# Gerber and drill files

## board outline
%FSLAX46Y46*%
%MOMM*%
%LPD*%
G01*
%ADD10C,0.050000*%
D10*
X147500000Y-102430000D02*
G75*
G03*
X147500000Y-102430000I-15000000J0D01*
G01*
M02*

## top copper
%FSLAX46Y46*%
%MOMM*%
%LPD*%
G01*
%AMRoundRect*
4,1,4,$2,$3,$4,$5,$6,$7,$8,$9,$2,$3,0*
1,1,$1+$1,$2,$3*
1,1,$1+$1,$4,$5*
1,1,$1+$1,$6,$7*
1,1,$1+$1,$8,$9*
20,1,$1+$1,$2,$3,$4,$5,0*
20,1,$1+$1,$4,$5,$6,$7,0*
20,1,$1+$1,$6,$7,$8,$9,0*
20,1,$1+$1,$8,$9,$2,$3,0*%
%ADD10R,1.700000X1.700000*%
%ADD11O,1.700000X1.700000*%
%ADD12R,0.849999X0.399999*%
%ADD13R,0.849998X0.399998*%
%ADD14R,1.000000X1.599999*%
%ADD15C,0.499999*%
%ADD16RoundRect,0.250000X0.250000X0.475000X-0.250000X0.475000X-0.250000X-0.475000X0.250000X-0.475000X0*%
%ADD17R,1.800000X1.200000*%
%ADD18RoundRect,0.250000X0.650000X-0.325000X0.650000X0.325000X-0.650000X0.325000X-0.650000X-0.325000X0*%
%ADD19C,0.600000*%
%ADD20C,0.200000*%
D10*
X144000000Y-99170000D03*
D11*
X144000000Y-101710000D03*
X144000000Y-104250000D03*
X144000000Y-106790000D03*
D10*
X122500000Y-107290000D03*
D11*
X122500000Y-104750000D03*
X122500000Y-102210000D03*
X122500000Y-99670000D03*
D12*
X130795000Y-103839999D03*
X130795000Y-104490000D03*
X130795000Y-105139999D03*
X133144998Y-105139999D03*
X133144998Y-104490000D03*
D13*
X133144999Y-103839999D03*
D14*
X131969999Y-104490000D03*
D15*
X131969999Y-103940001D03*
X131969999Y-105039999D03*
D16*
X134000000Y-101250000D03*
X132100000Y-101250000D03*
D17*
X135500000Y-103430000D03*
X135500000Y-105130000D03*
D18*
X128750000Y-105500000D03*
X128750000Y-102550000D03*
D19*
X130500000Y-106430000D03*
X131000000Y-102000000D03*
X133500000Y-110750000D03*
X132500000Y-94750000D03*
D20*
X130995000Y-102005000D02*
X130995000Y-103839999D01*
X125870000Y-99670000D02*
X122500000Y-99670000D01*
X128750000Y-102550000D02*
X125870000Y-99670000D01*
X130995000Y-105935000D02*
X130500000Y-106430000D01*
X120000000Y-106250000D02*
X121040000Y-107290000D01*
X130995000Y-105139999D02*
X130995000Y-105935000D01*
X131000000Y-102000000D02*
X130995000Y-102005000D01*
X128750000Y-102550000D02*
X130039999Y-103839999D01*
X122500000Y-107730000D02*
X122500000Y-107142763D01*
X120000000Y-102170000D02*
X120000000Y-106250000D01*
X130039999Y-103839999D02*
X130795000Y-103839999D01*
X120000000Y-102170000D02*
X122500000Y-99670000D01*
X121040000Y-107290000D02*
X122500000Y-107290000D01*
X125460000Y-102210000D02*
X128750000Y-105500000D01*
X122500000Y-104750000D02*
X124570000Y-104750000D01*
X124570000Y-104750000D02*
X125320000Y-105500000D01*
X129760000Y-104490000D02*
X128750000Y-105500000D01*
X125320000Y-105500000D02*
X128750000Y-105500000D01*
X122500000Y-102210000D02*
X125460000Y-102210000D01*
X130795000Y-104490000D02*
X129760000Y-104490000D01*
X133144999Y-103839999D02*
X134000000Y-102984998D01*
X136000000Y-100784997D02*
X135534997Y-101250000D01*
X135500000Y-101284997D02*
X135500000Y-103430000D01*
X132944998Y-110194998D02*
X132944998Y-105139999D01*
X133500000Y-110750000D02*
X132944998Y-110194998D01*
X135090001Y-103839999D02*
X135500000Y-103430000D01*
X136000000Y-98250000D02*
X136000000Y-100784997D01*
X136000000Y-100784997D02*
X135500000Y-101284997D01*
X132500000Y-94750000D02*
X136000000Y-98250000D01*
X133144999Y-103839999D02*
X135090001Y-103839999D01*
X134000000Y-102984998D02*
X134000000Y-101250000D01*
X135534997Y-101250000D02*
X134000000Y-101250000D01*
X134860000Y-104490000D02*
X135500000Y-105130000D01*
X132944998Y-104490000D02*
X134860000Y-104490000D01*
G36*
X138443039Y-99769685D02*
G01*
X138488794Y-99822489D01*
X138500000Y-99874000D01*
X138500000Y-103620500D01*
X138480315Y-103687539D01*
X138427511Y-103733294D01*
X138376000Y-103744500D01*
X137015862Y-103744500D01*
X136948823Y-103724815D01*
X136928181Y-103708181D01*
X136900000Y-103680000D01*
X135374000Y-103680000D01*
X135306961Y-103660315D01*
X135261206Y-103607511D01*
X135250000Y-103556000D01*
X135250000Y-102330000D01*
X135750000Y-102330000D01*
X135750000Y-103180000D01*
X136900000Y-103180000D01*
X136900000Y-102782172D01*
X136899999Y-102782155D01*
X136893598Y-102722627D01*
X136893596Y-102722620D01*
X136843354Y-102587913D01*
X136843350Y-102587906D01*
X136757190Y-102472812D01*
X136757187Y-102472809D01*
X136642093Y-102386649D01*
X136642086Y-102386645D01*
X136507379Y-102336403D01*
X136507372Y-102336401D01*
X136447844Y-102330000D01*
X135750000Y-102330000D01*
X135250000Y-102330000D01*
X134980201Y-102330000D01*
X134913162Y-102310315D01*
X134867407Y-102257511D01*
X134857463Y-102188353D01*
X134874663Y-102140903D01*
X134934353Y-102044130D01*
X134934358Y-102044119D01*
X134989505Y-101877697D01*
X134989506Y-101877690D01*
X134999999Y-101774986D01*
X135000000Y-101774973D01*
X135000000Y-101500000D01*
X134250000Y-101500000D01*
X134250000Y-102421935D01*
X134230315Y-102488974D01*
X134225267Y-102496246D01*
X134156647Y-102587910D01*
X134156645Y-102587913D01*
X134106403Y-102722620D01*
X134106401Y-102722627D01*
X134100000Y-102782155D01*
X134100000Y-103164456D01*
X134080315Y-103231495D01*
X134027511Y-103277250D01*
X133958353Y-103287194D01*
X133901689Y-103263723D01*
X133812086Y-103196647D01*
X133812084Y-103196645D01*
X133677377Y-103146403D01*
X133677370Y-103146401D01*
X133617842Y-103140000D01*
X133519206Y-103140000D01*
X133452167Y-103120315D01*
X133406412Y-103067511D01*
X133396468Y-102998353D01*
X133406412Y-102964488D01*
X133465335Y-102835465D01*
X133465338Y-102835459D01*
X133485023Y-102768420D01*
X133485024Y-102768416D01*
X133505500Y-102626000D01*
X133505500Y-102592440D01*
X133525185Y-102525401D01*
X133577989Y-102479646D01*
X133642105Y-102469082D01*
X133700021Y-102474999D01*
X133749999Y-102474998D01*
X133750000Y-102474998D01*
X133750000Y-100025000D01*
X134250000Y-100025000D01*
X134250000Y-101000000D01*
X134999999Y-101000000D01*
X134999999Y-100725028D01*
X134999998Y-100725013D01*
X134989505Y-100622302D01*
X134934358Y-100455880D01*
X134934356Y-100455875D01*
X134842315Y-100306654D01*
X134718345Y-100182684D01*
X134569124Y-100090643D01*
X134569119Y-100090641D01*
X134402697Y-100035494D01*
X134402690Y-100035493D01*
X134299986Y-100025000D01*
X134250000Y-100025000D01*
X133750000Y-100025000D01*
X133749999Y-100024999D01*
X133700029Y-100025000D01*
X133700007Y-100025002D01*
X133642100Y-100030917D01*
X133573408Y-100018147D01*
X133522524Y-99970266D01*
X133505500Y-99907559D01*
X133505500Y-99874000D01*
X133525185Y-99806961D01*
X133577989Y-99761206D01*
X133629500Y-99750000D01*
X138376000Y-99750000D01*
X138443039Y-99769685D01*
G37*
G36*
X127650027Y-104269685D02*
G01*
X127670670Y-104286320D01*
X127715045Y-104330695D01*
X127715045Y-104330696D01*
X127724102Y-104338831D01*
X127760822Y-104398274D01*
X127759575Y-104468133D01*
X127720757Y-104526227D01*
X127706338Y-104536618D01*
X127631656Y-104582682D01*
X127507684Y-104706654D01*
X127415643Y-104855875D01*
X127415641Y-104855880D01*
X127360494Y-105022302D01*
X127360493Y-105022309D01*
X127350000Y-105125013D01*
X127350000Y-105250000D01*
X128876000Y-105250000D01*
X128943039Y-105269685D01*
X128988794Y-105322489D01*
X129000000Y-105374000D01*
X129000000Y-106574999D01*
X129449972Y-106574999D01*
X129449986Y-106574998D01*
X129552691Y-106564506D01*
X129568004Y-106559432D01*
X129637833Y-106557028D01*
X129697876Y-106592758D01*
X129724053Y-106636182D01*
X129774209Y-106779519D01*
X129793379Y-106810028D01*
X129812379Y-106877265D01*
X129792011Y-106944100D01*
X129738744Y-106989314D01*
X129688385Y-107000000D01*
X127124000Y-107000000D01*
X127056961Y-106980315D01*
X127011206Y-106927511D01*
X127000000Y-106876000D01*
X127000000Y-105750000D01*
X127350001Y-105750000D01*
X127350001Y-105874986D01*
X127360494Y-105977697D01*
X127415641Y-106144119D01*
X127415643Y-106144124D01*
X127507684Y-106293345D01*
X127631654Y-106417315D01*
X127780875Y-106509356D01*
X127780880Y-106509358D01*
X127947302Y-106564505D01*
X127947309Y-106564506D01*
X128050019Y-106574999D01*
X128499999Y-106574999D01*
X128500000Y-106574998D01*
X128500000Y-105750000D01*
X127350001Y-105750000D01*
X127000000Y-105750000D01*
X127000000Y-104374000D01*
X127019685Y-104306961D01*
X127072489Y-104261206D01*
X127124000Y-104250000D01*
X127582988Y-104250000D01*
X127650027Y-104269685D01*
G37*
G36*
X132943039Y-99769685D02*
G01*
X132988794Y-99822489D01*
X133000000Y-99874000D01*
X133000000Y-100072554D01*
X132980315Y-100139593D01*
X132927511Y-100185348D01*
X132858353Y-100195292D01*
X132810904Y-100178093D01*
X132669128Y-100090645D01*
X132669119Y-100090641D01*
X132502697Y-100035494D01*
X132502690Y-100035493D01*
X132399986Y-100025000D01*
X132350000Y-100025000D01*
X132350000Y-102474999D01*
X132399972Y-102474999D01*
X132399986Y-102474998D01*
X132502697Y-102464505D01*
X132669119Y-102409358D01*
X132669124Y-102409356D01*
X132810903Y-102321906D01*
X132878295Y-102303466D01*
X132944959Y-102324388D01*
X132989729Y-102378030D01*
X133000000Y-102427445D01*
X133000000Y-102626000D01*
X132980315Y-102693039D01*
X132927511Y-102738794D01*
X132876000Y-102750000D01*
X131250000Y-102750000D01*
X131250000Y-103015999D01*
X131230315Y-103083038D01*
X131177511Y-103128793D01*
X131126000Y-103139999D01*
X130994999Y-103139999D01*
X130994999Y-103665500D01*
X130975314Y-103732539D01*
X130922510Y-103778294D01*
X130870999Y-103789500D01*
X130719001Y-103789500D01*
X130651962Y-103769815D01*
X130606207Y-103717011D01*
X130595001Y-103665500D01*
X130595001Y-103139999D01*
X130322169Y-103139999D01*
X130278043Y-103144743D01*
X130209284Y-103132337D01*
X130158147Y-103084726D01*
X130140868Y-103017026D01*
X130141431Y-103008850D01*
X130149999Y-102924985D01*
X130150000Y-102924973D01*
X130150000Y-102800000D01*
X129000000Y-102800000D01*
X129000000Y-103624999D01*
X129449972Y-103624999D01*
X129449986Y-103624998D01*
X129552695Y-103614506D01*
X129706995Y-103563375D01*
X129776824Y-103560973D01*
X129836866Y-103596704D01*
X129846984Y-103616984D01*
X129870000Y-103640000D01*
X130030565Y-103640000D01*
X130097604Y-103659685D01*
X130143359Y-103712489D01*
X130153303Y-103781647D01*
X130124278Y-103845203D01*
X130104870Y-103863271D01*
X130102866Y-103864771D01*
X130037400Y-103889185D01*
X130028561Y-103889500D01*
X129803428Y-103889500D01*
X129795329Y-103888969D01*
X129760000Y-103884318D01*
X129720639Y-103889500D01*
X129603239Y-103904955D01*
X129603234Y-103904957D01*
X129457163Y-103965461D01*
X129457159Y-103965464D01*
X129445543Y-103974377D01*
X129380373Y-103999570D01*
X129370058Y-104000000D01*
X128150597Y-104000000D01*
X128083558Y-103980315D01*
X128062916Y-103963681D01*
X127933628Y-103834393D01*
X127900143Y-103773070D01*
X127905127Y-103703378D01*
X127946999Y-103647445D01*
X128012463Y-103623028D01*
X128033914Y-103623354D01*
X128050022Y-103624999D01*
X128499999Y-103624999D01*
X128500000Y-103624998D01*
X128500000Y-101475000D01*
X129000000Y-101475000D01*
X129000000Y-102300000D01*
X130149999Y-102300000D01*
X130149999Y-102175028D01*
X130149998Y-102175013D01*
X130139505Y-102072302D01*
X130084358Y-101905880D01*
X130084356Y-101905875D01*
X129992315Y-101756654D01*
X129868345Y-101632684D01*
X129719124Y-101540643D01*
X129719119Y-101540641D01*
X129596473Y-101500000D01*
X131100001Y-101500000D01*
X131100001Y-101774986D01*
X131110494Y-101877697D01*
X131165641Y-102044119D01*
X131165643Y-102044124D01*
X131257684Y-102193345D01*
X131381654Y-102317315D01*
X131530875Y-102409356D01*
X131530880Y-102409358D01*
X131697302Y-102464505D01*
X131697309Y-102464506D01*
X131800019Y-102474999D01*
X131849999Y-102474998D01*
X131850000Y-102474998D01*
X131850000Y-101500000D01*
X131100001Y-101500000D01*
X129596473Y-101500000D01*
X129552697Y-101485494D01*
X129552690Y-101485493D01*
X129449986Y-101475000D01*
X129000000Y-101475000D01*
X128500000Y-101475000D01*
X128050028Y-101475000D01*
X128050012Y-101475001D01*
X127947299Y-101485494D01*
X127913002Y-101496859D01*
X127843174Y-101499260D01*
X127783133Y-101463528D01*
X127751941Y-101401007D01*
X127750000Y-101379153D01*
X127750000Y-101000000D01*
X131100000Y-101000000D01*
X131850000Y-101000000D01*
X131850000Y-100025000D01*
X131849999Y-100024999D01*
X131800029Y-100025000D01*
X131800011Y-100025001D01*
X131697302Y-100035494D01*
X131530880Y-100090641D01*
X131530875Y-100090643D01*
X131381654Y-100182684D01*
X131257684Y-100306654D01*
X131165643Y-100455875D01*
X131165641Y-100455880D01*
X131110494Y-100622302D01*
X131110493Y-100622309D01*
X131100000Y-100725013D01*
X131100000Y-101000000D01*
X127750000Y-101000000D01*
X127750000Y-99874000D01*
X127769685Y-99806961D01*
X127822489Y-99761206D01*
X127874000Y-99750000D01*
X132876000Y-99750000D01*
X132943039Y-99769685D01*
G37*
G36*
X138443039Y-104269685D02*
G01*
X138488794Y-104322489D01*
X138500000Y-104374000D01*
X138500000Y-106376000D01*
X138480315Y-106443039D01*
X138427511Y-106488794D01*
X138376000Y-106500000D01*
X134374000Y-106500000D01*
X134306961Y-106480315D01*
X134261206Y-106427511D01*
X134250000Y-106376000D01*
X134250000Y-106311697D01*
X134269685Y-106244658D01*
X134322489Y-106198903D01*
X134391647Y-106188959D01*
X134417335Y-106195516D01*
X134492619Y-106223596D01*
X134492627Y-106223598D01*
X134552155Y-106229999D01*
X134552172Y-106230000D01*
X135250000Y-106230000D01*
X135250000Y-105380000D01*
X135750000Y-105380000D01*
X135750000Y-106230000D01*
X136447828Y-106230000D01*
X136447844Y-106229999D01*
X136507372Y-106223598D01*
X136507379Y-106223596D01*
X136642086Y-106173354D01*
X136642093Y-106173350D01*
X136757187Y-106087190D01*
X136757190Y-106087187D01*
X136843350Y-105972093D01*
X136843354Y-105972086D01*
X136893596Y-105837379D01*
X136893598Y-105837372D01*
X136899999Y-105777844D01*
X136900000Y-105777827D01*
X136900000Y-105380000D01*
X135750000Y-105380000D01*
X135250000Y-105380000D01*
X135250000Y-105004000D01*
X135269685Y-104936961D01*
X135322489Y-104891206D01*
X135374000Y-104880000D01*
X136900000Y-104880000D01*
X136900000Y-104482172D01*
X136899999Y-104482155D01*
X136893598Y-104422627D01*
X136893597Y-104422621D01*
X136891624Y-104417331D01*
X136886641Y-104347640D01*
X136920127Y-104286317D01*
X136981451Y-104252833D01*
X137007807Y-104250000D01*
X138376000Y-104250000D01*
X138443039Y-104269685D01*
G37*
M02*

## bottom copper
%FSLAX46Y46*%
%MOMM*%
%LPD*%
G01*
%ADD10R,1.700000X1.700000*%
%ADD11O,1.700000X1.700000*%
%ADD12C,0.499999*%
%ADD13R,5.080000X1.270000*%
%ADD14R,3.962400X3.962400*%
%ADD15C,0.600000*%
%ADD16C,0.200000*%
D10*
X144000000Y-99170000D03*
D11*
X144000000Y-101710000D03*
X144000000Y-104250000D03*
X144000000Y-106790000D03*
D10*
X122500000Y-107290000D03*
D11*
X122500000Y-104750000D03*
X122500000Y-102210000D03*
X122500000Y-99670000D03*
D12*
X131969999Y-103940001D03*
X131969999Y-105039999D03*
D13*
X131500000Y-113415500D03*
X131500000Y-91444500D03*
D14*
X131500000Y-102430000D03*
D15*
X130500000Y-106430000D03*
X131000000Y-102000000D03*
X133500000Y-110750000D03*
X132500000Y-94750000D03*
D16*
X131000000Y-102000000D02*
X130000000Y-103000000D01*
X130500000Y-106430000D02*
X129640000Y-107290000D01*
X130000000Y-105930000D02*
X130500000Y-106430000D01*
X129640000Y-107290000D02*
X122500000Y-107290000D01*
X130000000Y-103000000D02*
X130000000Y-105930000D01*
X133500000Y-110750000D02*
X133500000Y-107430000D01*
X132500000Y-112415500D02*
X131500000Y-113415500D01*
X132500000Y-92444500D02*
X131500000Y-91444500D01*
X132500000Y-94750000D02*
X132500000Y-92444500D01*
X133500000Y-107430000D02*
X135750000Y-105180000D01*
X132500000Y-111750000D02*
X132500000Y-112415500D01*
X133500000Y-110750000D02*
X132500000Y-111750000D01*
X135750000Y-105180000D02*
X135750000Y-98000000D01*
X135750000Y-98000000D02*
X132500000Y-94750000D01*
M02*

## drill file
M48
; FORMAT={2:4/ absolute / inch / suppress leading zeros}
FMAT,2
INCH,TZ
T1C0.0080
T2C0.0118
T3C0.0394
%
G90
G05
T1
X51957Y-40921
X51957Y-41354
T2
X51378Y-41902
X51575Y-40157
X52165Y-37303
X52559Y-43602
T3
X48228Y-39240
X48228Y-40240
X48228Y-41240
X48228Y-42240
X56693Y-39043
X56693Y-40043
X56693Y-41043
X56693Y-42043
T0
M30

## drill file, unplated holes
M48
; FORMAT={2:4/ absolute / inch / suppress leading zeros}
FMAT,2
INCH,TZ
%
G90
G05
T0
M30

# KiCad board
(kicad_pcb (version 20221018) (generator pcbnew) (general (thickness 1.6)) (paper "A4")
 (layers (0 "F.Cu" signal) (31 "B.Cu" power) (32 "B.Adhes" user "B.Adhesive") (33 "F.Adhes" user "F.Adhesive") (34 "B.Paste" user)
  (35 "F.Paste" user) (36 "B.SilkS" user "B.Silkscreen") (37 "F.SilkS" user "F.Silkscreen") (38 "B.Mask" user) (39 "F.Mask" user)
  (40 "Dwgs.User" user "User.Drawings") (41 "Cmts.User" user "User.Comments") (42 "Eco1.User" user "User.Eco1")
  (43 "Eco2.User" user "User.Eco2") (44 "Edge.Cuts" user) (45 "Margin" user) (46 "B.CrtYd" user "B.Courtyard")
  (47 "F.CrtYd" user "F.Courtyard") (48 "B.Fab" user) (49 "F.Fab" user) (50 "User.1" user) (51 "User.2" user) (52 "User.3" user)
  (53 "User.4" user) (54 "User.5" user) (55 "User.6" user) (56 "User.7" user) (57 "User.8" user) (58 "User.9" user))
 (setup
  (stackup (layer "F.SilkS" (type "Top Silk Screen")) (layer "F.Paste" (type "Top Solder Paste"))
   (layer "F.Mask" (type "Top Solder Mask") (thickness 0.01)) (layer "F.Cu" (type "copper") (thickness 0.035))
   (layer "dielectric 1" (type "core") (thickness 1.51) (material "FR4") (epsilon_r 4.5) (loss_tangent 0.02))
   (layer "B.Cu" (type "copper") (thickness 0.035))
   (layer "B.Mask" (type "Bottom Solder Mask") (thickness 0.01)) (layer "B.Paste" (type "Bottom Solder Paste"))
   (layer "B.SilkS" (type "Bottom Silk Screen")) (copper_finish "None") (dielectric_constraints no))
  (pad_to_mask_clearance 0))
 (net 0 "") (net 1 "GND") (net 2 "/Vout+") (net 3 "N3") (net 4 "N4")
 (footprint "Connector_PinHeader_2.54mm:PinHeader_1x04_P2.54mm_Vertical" (layer "F.Cu") (at 144 99.17)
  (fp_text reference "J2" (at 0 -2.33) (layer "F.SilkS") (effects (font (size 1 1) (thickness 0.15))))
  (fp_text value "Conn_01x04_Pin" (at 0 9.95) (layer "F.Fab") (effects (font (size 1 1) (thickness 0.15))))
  (pad "1" thru_hole rect (at 0 0) (size 1.7 1.7) (drill 1) (layers "*.Cu" "*.Mask"))
  (pad "2" thru_hole oval (at 0 2.54) (size 1.7 1.7) (drill 1) (layers "*.Cu" "*.Mask"))
  (pad "3" thru_hole oval (at 0 5.08) (size 1.7 1.7) (drill 1) (layers "*.Cu" "*.Mask"))
  (pad "4" thru_hole oval (at 0 7.62) (size 1.7 1.7) (drill 1) (layers "*.Cu" "*.Mask")))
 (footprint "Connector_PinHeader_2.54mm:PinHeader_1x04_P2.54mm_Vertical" (layer "F.Cu") (at 122.5 107.29 180)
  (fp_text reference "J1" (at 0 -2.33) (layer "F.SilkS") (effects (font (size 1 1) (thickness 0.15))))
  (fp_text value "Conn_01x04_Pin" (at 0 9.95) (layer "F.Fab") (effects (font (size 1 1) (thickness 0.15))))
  (pad "1" thru_hole rect (at 0 0 180) (size 1.7 1.7) (drill 1) (layers "*.Cu" "*.Mask") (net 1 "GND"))
  (pad "2" thru_hole oval (at 0 2.54 180) (size 1.7 1.7) (drill 1) (layers "*.Cu" "*.Mask") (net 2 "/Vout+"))
  (pad "3" thru_hole oval (at 0 5.08 180) (size 1.7 1.7) (drill 1) (layers "*.Cu" "*.Mask") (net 2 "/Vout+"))
  (pad "4" thru_hole oval (at 0 7.62 180) (size 1.7 1.7) (drill 1) (layers "*.Cu" "*.Mask") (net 1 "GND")))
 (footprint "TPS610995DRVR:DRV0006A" (layer "F.Cu") (at 131.969999 104.49)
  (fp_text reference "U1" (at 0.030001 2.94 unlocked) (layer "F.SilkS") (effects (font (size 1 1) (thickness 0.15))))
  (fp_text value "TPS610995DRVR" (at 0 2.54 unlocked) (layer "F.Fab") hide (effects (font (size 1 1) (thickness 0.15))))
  (pad "1" smd rect (at -1.174999 -0.650001 90) (size 0.399999 0.849999) (layers "F.Cu" "F.Paste" "F.Mask") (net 1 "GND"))
  (pad "2" smd rect (at -1.174999 0 90) (size 0.399999 0.849999) (layers "F.Cu" "F.Paste" "F.Mask") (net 2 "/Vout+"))
  (pad "3" smd rect (at -1.174999 0.649999 90) (size 0.399999 0.849999) (layers "F.Cu" "F.Paste" "F.Mask") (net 1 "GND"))
  (pad "4" smd rect (at 1.174999 0.649999 90) (size 0.399999 0.849999) (layers "F.Cu" "F.Paste" "F.Mask") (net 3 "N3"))
  (pad "5" smd rect (at 1.174999 0 90) (size 0.399999 0.849999) (layers "F.Cu" "F.Paste" "F.Mask") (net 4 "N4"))
  (pad "6" smd rect (at 1.175 -0.650001 90) (size 0.399998 0.849998) (layers "F.Cu" "F.Paste" "F.Mask") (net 3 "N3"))
  (pad "7" smd rect (at 0 0) (size 1 1.599999) (layers "F.Cu" "F.Paste" "F.Mask") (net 1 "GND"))
  (pad "V" thru_hole circle (at 0 -0.549999) (size 0.499999 0.499999) (drill 0.2032) (layers "*.Cu" "*.Mask") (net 1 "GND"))
  (pad "V" thru_hole circle (at 0 0.549999) (size 0.499999 0.499999) (drill 0.2032) (layers "*.Cu" "*.Mask") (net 1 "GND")))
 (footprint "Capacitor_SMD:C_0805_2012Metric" (layer "F.Cu") (at 133.05 101.25 180)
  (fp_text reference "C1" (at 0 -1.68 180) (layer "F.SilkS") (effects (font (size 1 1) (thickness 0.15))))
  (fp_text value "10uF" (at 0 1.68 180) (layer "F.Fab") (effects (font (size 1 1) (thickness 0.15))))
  (pad "1" smd roundrect (at -0.95 0 180) (size 1 1.45) (layers "F.Cu" "F.Paste" "F.Mask") (roundrect_rratio 0.25) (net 3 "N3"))
  (pad "2" smd roundrect (at 0.95 0 180) (size 1 1.45) (layers "F.Cu" "F.Paste" "F.Mask") (roundrect_rratio 0.25) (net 1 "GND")))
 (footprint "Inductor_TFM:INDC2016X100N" (layer "F.Cu") (at 135.5 104.28 -90)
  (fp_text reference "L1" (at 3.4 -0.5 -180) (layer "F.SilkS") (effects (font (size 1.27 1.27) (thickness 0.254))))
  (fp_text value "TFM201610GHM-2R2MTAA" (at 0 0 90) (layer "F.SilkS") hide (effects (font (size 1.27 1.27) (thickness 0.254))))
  (pad "1" smd rect (at -0.85 0 270) (size 1.2 1.8) (layers "F.Cu" "F.Paste" "F.Mask") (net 3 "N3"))
  (pad "2" smd rect (at 0.85 0 270) (size 1.2 1.8) (layers "F.Cu" "F.Paste" "F.Mask") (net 4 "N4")))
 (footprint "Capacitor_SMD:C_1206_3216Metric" (layer "F.Cu") (at 128.75 104.025 90)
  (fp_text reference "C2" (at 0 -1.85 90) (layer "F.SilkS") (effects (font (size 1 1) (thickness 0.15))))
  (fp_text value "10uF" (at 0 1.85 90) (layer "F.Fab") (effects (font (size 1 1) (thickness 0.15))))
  (pad "1" smd roundrect (at -1.475 0 90) (size 1.15 1.8) (layers "F.Cu" "F.Paste" "F.Mask") (roundrect_rratio 0.217391) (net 2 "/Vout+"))
  (pad "2" smd roundrect (at 1.475 0 90) (size 1.15 1.8) (layers "F.Cu" "F.Paste" "F.Mask") (roundrect_rratio 0.217391) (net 1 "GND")))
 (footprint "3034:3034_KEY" (layer "B.Cu") (at 132.1731 102.43 90)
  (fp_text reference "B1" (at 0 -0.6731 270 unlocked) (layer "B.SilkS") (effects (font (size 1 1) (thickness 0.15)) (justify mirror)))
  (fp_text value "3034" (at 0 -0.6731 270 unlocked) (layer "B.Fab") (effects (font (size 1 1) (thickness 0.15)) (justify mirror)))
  (pad "1" smd rect (at -10.9855 -0.6731 90) (size 1.27 5.08) (layers "B.Cu" "B.Paste" "B.Mask") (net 3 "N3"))
  (pad "2" smd rect (at 10.9855 -0.6731 90) (size 1.27 5.08) (layers "B.Cu" "B.Paste" "B.Mask") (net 3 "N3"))
  (pad "3" smd rect (at 0 -0.6731 90) (size 3.9624 3.9624) (layers "B.Cu" "B.Paste" "B.Mask") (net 1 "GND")))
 (gr_circle (center 132.5 102.43) (end 141.5 114.43) (stroke (width 0.05) (type default)) (fill none) (layer "Edge.Cuts"))
 (segment (start 130.995 102.005) (end 130.995 103.839999) (width 0.2) (layer "F.Cu") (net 1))
 (segment (start 125.87 99.67) (end 122.5 99.67) (width 0.2) (layer "F.Cu") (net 1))
 (segment (start 128.75 102.55) (end 125.87 99.67) (width 0.2) (layer "F.Cu") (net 1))
 (segment (start 130.995 105.935) (end 130.5 106.43) (width 0.2) (layer "F.Cu") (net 1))
 (segment (start 120 106.25) (end 121.04 107.29) (width 0.2) (layer "F.Cu") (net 1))
 (segment (start 130.995 105.139999) (end 130.995 105.935) (width 0.2) (layer "F.Cu") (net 1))
 (segment (start 131 102) (end 130.995 102.005) (width 0.2) (layer "F.Cu") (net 1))
 (segment (start 128.75 102.55) (end 130.039999 103.839999) (width 0.2) (layer "F.Cu") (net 1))
 (segment (start 122.5 107.73) (end 122.5 107.142763) (width 0.2) (layer "F.Cu") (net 1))
 (segment (start 120 102.17) (end 120 106.25) (width 0.2) (layer "F.Cu") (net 1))
 (segment (start 130.039999 103.839999) (end 130.795 103.839999) (width 0.2) (layer "F.Cu") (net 1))
 (segment (start 120 102.17) (end 122.5 99.67) (width 0.2) (layer "F.Cu") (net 1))
 (segment (start 121.04 107.29) (end 122.5 107.29) (width 0.2) (layer "F.Cu") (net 1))
 (via (at 130.5 106.43) (size 0.6) (drill 0.3) (layers "F.Cu" "B.Cu") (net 1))
 (via (at 131 102) (size 0.6) (drill 0.3) (layers "F.Cu" "B.Cu") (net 1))
 (segment (start 131 102) (end 130 103) (width 0.2) (layer "B.Cu") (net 1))
 (segment (start 130.5 106.43) (end 129.64 107.29) (width 0.2) (layer "B.Cu") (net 1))
 (segment (start 130 105.93) (end 130.5 106.43) (width 0.2) (layer "B.Cu") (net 1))
 (segment (start 129.64 107.29) (end 122.5 107.29) (width 0.2) (layer "B.Cu") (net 1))
 (segment (start 130 103) (end 130 105.93) (width 0.2) (layer "B.Cu") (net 1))
 (segment (start 125.46 102.21) (end 128.75 105.5) (width 0.2) (layer "F.Cu") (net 2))
 (segment (start 122.5 104.75) (end 124.57 104.75) (width 0.2) (layer "F.Cu") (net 2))
 (segment (start 124.57 104.75) (end 125.32 105.5) (width 0.2) (layer "F.Cu") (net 2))
 (segment (start 129.76 104.49) (end 128.75 105.5) (width 0.2) (layer "F.Cu") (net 2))
 (segment (start 125.32 105.5) (end 128.75 105.5) (width 0.2) (layer "F.Cu") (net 2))
 (segment (start 122.5 102.21) (end 125.46 102.21) (width 0.2) (layer "F.Cu") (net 2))
 (segment (start 130.795 104.49) (end 129.76 104.49) (width 0.2) (layer "F.Cu") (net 2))
 (segment (start 133.144999 103.839999) (end 134 102.984998) (width 0.2) (layer "F.Cu") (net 3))
 (segment (start 136 100.784997) (end 135.534997 101.25) (width 0.2) (layer "F.Cu") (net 3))
 (segment (start 135.5 101.284997) (end 135.5 103.43) (width 0.2) (layer "F.Cu") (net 3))
 (segment (start 132.944998 110.194998) (end 132.944998 105.139999) (width 0.2) (layer "F.Cu") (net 3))
 (segment (start 133.5 110.75) (end 132.944998 110.194998) (width 0.2) (layer "F.Cu") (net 3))
 (segment (start 135.090001 103.839999) (end 135.5 103.43) (width 0.2) (layer "F.Cu") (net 3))
 (segment (start 136 98.25) (end 136 100.784997) (width 0.2) (layer "F.Cu") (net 3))
 (segment (start 136 100.784997) (end 135.5 101.284997) (width 0.2) (layer "F.Cu") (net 3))
 (segment (start 132.5 94.75) (end 136 98.25) (width 0.2) (layer "F.Cu") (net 3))
 (segment (start 133.144999 103.839999) (end 135.090001 103.839999) (width 0.2) (layer "F.Cu") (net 3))
 (segment (start 134 102.984998) (end 134 101.25) (width 0.2) (layer "F.Cu") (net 3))
 (segment (start 135.534997 101.25) (end 134 101.25) (width 0.2) (layer "F.Cu") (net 3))
 (via (at 133.5 110.75) (size 0.6) (drill 0.3) (layers "F.Cu" "B.Cu") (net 3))
 (via (at 132.5 94.75) (size 0.6) (drill 0.3) (layers "F.Cu" "B.Cu") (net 3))
 (segment (start 133.5 110.75) (end 133.5 107.43) (width 0.2) (layer "B.Cu") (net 3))
 (segment (start 132.5 112.4155) (end 131.5 113.4155) (width 0.2) (layer "B.Cu") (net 3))
 (segment (start 132.5 92.4445) (end 131.5 91.4445) (width 0.2) (layer "B.Cu") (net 3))
 (segment (start 132.5 94.75) (end 132.5 92.4445) (width 0.2) (layer "B.Cu") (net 3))
 (segment (start 133.5 107.43) (end 135.75 105.18) (width 0.2) (layer "B.Cu") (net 3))
 (segment (start 132.5 111.75) (end 132.5 112.4155) (width 0.2) (layer "B.Cu") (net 3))
 (segment (start 133.5 110.75) (end 132.5 111.75) (width 0.2) (layer "B.Cu") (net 3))
 (segment (start 135.75 105.18) (end 135.75 98) (width 0.2) (layer "B.Cu") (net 3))
 (segment (start 135.75 98) (end 132.5 94.75) (width 0.2) (layer "B.Cu") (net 3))
 (segment (start 134.86 104.49) (end 135.5 105.13) (width 0.2) (layer "F.Cu") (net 4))
 (segment (start 132.944998 104.49) (end 134.86 104.49) (width 0.2) (layer "F.Cu") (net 4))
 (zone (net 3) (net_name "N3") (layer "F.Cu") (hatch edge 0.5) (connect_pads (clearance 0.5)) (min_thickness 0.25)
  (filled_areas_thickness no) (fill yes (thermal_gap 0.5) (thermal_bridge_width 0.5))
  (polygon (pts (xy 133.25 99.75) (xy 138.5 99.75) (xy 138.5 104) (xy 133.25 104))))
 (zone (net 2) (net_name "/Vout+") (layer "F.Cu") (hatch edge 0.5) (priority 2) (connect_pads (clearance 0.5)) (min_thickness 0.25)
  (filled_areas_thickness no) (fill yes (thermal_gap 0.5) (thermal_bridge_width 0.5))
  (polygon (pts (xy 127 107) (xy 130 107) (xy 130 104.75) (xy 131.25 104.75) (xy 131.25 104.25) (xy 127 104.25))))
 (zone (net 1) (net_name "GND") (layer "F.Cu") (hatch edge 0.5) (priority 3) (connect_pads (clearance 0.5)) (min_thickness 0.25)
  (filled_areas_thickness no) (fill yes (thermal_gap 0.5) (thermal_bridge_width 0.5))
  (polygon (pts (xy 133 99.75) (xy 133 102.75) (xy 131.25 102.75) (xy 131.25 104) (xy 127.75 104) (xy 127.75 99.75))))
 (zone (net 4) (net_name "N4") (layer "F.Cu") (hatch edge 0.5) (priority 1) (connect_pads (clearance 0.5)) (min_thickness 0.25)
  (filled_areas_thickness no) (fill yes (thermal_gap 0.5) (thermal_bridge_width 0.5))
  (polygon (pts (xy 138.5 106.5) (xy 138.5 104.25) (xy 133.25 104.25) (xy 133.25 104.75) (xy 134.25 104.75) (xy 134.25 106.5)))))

